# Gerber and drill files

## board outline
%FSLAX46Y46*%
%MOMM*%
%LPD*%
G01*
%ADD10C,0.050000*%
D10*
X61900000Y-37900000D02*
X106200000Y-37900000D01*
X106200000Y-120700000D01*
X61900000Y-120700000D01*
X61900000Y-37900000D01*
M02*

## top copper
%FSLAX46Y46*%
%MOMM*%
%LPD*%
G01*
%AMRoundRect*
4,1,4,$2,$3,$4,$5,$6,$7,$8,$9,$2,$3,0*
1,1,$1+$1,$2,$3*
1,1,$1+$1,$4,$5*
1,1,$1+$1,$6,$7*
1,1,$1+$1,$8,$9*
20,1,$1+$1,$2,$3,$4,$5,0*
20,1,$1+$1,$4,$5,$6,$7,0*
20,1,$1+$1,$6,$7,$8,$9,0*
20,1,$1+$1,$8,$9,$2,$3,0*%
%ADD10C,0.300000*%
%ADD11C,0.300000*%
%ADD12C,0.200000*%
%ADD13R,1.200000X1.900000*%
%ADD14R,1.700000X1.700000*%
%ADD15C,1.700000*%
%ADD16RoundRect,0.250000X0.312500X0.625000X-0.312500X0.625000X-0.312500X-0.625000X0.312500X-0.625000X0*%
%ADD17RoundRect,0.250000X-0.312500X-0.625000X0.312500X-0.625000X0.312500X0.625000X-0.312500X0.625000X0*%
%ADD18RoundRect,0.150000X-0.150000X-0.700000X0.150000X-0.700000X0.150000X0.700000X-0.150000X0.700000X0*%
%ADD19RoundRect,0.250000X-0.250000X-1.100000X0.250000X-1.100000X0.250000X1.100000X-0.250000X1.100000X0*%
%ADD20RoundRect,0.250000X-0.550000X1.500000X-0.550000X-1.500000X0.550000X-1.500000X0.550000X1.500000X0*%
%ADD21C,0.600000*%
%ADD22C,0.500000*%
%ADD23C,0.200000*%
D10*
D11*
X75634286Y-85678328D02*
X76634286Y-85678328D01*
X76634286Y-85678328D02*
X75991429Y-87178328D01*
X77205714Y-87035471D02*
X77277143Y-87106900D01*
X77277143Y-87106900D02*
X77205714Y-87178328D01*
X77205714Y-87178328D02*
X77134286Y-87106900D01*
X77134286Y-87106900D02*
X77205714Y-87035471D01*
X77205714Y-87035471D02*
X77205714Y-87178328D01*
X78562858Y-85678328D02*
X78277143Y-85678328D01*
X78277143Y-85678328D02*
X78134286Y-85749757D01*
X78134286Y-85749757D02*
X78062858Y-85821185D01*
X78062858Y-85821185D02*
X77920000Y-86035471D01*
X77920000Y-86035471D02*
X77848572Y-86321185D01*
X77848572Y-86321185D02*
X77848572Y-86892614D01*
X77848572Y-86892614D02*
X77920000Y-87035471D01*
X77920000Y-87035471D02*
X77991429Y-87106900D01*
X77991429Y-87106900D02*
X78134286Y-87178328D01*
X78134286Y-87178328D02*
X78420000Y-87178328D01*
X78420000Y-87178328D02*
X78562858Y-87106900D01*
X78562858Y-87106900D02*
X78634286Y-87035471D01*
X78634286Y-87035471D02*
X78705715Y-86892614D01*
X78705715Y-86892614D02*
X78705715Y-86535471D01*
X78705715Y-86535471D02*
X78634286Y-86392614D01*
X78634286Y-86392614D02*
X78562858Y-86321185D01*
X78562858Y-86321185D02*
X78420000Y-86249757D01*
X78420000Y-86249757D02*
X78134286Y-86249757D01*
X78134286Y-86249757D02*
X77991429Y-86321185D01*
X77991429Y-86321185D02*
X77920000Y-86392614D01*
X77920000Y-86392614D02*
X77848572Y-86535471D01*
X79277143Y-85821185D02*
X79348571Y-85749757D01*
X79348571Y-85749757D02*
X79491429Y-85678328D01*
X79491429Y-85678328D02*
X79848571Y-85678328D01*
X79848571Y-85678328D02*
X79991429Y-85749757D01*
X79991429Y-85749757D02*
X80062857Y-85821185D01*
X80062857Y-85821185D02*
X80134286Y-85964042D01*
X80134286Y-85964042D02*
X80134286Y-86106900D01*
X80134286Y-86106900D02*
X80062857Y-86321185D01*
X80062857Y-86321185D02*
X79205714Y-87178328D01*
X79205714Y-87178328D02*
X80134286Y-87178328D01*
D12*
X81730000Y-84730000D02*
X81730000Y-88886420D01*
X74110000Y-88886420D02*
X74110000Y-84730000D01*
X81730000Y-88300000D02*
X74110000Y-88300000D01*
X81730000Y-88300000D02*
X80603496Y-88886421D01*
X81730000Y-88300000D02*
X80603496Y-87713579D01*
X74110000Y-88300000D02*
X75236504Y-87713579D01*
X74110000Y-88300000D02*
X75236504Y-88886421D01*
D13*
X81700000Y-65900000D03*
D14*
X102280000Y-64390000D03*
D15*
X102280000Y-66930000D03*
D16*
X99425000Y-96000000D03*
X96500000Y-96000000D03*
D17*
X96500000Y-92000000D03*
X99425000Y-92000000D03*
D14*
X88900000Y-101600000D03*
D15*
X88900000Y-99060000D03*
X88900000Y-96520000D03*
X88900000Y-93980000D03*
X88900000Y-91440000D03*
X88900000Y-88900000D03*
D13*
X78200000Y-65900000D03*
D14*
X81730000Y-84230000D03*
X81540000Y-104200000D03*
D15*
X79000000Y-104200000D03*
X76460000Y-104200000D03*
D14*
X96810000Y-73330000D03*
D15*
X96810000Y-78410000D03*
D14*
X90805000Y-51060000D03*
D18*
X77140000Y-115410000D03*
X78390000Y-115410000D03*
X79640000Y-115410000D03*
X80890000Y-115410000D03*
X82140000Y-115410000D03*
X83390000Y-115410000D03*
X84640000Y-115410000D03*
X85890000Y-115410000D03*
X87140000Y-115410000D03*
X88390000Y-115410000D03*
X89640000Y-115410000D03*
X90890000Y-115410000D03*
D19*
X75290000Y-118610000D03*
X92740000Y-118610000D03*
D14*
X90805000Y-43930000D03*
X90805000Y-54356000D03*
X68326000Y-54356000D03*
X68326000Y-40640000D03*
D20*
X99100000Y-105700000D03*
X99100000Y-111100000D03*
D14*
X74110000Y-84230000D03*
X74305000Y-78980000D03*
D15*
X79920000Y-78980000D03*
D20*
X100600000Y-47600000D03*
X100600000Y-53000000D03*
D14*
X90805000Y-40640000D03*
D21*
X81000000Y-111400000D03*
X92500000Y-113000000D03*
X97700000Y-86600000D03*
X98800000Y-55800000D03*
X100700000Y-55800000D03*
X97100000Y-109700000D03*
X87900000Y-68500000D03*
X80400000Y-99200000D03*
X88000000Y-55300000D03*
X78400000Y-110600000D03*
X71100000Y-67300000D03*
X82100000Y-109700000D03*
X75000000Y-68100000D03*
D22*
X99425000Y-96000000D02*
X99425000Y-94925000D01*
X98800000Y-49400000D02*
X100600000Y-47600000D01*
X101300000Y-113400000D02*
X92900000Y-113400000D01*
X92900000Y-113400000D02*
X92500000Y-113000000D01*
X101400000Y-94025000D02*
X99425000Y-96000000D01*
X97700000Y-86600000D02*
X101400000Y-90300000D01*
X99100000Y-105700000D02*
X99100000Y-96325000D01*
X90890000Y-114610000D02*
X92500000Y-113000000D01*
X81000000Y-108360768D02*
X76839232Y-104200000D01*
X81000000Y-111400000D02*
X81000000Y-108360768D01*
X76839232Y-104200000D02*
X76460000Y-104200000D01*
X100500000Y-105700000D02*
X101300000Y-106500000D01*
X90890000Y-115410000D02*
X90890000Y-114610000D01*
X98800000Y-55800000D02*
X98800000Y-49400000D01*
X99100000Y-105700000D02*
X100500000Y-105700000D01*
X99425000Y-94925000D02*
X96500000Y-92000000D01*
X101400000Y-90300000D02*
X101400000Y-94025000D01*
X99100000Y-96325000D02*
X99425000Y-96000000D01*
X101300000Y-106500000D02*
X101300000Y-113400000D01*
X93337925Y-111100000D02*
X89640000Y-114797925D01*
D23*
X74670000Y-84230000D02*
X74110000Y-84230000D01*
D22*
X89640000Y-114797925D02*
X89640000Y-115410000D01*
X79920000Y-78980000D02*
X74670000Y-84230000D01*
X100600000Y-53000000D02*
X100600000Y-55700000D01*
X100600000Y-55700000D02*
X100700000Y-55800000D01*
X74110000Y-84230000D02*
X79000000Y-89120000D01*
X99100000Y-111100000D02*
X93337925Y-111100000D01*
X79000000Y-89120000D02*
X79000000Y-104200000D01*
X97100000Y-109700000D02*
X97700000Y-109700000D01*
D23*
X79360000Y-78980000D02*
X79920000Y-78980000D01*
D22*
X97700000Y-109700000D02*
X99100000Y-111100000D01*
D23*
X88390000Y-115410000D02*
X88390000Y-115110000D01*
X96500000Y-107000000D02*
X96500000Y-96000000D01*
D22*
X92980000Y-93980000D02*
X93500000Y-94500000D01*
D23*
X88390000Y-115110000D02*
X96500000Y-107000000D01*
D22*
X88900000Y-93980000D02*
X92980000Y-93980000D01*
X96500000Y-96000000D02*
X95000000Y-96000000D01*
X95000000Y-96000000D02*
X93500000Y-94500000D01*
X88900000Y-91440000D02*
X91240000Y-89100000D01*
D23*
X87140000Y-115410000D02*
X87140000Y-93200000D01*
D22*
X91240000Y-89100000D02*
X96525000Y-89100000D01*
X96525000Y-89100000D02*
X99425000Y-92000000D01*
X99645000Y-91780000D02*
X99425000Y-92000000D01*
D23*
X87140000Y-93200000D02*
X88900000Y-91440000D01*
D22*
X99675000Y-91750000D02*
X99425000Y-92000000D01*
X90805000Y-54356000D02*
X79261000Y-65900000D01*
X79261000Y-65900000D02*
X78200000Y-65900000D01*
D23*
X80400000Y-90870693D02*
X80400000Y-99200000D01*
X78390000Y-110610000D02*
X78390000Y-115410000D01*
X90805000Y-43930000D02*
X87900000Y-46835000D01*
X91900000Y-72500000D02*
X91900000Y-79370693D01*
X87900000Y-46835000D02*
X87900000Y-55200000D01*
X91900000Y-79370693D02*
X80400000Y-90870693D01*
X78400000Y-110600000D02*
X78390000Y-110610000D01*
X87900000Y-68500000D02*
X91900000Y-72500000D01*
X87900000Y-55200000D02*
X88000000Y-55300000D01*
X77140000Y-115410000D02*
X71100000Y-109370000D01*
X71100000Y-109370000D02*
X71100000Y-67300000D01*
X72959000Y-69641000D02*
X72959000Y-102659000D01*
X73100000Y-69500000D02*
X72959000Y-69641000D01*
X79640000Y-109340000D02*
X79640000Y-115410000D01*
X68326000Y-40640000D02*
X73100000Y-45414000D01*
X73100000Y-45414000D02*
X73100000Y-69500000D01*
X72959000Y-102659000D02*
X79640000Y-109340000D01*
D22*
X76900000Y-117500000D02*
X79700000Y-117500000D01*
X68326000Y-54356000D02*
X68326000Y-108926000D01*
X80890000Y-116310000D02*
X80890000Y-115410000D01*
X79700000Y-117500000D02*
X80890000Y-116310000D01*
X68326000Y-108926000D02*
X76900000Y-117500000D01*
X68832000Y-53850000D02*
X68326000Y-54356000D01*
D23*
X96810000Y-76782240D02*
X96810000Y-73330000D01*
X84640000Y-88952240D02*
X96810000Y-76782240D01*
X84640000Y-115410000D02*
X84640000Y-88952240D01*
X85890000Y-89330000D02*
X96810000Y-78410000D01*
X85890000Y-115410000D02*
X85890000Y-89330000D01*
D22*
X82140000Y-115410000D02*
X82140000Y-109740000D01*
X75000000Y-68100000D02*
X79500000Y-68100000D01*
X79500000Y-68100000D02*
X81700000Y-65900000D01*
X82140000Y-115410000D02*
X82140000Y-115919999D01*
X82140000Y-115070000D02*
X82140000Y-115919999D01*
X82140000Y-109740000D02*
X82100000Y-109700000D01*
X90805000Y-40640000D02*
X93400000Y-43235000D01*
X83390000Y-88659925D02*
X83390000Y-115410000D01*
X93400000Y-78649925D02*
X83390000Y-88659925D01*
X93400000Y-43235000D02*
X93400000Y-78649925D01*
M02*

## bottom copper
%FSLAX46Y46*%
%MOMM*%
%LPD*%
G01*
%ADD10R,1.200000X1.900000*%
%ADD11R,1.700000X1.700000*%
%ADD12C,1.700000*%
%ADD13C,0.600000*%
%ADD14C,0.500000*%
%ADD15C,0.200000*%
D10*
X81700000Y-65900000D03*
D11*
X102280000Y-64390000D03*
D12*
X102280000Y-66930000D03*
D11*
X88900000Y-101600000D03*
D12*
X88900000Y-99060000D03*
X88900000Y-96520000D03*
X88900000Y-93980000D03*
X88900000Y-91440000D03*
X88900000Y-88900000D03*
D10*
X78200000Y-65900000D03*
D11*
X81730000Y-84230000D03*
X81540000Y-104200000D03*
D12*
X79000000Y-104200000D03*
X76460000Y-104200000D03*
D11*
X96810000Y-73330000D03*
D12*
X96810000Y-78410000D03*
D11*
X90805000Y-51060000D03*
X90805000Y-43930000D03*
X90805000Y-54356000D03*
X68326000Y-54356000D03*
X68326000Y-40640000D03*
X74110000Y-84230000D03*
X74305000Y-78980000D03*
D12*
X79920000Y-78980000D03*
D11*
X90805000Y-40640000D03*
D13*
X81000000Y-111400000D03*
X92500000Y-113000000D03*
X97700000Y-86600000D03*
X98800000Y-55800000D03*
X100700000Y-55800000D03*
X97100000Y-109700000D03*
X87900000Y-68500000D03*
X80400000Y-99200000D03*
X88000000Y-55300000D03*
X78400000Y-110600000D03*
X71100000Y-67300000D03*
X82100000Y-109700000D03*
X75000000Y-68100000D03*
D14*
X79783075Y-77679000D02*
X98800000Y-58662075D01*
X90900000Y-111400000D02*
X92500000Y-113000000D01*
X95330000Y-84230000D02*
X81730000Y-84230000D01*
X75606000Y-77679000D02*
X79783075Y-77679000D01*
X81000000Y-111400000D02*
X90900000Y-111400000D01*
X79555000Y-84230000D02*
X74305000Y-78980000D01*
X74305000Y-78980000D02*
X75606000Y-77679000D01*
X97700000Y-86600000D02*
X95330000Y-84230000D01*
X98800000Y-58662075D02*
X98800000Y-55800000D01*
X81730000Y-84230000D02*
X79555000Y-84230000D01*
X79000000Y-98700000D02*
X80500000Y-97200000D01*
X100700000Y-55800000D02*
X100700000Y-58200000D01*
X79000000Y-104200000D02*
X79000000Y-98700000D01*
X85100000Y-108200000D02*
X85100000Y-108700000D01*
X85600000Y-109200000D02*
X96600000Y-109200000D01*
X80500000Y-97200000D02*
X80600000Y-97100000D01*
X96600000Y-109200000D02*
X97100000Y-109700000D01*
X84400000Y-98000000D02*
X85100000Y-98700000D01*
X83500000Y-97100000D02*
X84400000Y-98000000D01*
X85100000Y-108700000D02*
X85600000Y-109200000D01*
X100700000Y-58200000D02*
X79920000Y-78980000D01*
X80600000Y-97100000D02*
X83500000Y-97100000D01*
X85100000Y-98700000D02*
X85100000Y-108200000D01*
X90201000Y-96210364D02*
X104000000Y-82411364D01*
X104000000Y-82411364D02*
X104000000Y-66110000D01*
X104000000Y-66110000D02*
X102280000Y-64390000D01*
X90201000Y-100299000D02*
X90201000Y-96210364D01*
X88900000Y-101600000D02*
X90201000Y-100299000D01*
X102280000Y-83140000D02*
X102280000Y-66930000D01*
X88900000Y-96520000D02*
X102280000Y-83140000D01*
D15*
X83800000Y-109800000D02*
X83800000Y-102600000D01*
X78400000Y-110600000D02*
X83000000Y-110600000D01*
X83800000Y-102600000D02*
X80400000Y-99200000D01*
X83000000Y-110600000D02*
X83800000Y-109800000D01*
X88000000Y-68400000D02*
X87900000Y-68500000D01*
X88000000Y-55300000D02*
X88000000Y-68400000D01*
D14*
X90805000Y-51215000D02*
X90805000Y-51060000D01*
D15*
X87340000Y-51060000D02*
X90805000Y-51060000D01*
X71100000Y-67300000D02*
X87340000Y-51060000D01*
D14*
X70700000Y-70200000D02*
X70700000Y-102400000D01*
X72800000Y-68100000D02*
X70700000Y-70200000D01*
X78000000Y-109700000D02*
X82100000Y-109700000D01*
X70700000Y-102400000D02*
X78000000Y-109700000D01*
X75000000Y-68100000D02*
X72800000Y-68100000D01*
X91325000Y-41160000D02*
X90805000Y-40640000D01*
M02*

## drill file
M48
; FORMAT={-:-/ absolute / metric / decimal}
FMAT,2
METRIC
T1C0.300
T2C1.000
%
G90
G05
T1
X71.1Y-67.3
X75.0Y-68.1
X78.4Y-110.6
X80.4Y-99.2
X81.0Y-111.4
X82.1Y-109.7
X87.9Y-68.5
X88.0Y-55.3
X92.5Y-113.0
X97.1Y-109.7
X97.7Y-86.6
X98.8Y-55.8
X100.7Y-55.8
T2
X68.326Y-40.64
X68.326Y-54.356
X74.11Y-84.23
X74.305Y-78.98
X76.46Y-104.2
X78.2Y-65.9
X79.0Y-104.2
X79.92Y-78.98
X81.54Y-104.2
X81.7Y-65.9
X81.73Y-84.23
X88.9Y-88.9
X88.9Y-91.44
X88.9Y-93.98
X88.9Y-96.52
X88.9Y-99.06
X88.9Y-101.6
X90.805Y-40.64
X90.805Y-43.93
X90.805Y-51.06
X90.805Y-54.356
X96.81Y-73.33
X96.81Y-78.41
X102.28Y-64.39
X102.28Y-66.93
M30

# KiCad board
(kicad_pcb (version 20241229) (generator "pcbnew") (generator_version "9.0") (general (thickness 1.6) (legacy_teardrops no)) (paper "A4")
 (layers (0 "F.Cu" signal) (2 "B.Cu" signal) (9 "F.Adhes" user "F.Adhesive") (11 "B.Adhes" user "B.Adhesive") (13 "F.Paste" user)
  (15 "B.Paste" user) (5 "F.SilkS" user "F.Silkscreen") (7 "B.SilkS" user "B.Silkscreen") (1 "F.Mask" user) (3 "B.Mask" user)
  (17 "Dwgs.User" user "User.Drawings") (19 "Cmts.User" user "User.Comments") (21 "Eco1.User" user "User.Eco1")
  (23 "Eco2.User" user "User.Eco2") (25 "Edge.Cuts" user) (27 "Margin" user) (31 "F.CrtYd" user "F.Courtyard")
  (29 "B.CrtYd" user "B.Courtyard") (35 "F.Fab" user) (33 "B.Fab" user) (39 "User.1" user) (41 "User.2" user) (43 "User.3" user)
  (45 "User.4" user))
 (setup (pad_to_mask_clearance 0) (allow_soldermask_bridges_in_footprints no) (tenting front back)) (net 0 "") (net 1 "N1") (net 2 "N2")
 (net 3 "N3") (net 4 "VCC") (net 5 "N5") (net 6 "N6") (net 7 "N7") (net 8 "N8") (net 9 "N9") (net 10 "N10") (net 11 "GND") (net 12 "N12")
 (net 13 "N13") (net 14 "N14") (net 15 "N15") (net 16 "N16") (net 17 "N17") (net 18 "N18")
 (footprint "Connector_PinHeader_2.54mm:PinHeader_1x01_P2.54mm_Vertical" (layer "F.Cu") (at 81.7 65.9 90)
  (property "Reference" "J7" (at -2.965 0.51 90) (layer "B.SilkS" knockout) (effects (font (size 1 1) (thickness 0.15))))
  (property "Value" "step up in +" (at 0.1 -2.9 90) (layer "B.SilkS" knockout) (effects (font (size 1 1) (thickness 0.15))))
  (pad "1" thru_hole rect (at 0 0 90) (size 1.9 1.2) (drill 1) (layers "*.Cu" "*.Mask") (remove_unused_layers no) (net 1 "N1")))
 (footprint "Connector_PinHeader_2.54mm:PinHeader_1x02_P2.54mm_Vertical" (layer "F.Cu") (at 102.28 64.39)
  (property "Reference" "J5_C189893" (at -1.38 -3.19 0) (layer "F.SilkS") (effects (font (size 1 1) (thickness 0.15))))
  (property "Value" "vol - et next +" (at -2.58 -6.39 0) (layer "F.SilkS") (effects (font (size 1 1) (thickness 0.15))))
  (pad "1" thru_hole rect (at 0 0) (size 1.7 1.7) (drill 1) (layers "*.Cu" "*.Mask") (remove_unused_layers no) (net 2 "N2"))
  (pad "2" thru_hole circle (at 0 2.54) (size 1.7 1.7) (drill 1) (layers "*.Cu" "*.Mask") (remove_unused_layers no) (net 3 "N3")))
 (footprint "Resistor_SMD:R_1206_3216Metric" (layer "F.Cu") (at 97.9625 96 180)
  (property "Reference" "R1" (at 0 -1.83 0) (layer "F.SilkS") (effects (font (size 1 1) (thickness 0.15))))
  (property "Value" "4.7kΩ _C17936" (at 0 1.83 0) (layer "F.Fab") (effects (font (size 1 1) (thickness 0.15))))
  (pad "1" smd roundrect (at -1.4625 0 180) (size 1.125 1.75) (layers "F.Cu" "F.Mask" "F.Paste") (roundrect_rratio 0.222222) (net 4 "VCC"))
  (pad "2" smd roundrect (at 1.4625 0 180) (size 1.125 1.75) (layers "F.Cu" "F.Mask" "F.Paste") (roundrect_rratio 0.222222) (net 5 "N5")))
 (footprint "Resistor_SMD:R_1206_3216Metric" (layer "F.Cu") (at 97.9625 92)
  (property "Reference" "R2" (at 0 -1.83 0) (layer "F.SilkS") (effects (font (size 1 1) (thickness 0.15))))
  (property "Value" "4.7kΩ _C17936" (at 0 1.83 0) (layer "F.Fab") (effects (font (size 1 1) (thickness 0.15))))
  (pad "1" smd roundrect (at -1.4625 0) (size 1.125 1.75) (layers "F.Cu" "F.Mask" "F.Paste") (roundrect_rratio 0.222222) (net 4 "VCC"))
  (pad "2" smd roundrect (at 1.4625 0) (size 1.125 1.75) (layers "F.Cu" "F.Mask" "F.Paste") (roundrect_rratio 0.222222) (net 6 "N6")))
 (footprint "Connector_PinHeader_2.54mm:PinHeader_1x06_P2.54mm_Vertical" (layer "F.Cu") (at 88.9 101.6 180)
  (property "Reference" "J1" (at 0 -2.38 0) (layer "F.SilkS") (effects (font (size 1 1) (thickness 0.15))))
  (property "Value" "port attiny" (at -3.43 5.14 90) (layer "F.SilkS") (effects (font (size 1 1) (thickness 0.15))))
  (pad "1" thru_hole rect (at 0 0 180) (size 1.7 1.7) (drill 1) (layers "*.Cu" "*.Mask") (remove_unused_layers no) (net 2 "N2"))
  (pad "2" thru_hole circle (at 0 2.54 180) (size 1.7 1.7) (drill 1) (layers "*.Cu" "*.Mask") (remove_unused_layers no) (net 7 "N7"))
  (pad "3" thru_hole circle (at 0 5.08 180) (size 1.7 1.7) (drill 1) (layers "*.Cu" "*.Mask") (remove_unused_layers no) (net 3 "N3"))
  (pad "4" thru_hole circle (at 0 7.62 180) (size 1.7 1.7) (drill 1) (layers "*.Cu" "*.Mask") (remove_unused_layers no) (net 5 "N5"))
  (pad "5" thru_hole circle (at 0 10.16 180) (size 1.7 1.7) (drill 1) (layers "*.Cu" "*.Mask") (remove_unused_layers no) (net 6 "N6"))
  (pad "6" thru_hole circle (at 0 12.7 180) (size 1.7 1.7) (drill 1) (layers "*.Cu" "*.Mask") (remove_unused_layers no) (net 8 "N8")))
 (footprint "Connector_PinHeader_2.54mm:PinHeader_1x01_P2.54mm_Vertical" (layer "F.Cu") (at 78.1 65.9 90)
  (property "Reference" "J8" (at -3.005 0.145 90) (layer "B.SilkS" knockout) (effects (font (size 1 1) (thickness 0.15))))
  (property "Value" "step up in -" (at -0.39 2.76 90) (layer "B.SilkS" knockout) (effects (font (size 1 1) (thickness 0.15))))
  (pad "1" thru_hole rect (at 0 0.1 90) (size 1.9 1.2) (drill 1) (layers "*.Cu" "*.Mask") (remove_unused_layers no) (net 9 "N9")))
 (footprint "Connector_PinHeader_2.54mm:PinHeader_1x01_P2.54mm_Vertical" (layer "F.Cu") (at 81.73 84.23)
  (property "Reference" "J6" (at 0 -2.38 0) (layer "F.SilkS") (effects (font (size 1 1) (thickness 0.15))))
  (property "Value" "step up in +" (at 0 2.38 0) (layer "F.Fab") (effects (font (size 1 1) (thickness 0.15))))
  (pad "1" thru_hole rect (at 0 0) (size 1.7 1.7) (drill 1) (layers "*.Cu" "*.Mask") (remove_unused_layers no) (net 4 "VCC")
   (padstack (mode custom) (layer "B.Cu" (shape rect) (size 1.7 1.7) (zone_connect -1)))))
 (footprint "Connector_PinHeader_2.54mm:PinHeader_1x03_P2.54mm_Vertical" (layer "F.Cu") (at 81.54 104.2 -90)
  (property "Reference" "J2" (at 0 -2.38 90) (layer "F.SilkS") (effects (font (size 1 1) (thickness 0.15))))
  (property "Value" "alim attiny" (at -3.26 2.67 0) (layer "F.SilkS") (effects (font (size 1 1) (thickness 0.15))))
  (pad "1" thru_hole rect (at 0 0 270) (size 1.7 1.7) (drill 1) (layers "*.Cu" "*.Mask") (remove_unused_layers no) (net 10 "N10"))
  (pad "2" thru_hole circle (at 0 2.54 270) (size 1.7 1.7) (drill 1) (layers "*.Cu" "*.Mask") (remove_unused_layers no) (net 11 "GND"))
  (pad "3" thru_hole circle (at 0 5.08 270) (size 1.7 1.7) (drill 1) (layers "*.Cu" "*.Mask") (remove_unused_layers no) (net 4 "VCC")))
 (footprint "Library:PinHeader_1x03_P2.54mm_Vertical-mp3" (layer "F.Cu") (at 96.81 73.33)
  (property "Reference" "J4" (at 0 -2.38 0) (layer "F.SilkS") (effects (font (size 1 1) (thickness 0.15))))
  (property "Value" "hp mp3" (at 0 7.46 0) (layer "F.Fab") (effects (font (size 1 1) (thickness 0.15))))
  (pad "1" thru_hole rect (at 0 0) (size 1.7 1.7) (drill 1) (layers "*.Cu" "*.Mask") (remove_unused_layers no) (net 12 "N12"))
  (pad "2" thru_hole circle (at 0 5.08) (size 1.7 1.7) (drill 1) (layers "*.Cu" "*.Mask") (remove_unused_layers no) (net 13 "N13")))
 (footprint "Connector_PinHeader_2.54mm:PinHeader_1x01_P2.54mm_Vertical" (layer "F.Cu") (at 90.805 51.06)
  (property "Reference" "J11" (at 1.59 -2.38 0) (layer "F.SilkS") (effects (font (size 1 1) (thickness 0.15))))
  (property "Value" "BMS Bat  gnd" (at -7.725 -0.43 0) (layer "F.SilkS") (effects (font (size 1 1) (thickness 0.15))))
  (pad "1" thru_hole rect (at 0 0) (size 1.7 1.7) (drill 1) (layers "*.Cu" "*.Mask") (remove_unused_layers no) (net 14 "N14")))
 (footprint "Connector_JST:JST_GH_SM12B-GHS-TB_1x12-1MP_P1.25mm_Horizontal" (layer "F.Cu") (at 84.015 117.26)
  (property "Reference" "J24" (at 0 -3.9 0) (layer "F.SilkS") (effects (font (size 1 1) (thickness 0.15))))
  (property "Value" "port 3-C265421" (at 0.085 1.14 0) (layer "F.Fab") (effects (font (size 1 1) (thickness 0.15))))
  (pad "1" smd roundrect (at -6.875 -1.85) (size 0.6 1.7) (layers "F.Cu" "F.Mask" "F.Paste") (roundrect_rratio 0.25) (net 14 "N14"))
  (pad "2" smd roundrect (at -5.625 -1.85) (size 0.6 1.7) (layers "F.Cu" "F.Mask" "F.Paste") (roundrect_rratio 0.25) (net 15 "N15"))
  (pad "3" smd roundrect (at -4.375 -1.85) (size 0.6 1.7) (layers "F.Cu" "F.Mask" "F.Paste") (roundrect_rratio 0.25) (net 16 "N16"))
  (pad "4" smd roundrect (at -3.125 -1.85) (size 0.6 1.7) (layers "F.Cu" "F.Mask" "F.Paste") (roundrect_rratio 0.25) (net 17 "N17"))
  (pad "5" smd roundrect (at -1.875 -1.85) (size 0.6 1.7) (layers "F.Cu" "F.Mask" "F.Paste") (roundrect_rratio 0.25) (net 1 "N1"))
  (pad "6" smd roundrect (at -0.625 -1.85) (size 0.6 1.7) (layers "F.Cu" "F.Mask" "F.Paste") (roundrect_rratio 0.25) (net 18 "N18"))
  (pad "7" smd roundrect (at 0.625 -1.85) (size 0.6 1.7) (layers "F.Cu" "F.Mask" "F.Paste") (roundrect_rratio 0.25) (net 12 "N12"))
  (pad "8" smd roundrect (at 1.875 -1.85) (size 0.6 1.7) (layers "F.Cu" "F.Mask" "F.Paste") (roundrect_rratio 0.25) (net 13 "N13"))
  (pad "9" smd roundrect (at 3.125 -1.85) (size 0.6 1.7) (layers "F.Cu" "F.Mask" "F.Paste") (roundrect_rratio 0.25) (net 6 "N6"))
  (pad "10" smd roundrect (at 4.375 -1.85) (size 0.6 1.7) (layers "F.Cu" "F.Mask" "F.Paste") (roundrect_rratio 0.25) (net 5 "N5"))
  (pad "11" smd roundrect (at 5.625 -1.85) (size 0.6 1.7) (layers "F.Cu" "F.Mask" "F.Paste") (roundrect_rratio 0.25) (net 11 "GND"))
  (pad "12" smd roundrect (at 6.875 -1.85) (size 0.6 1.7) (layers "F.Cu" "F.Mask" "F.Paste") (roundrect_rratio 0.25) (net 4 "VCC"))
  (pad "MP" smd roundrect (at -8.725 1.35) (size 1 2.7) (layers "F.Cu" "F.Mask" "F.Paste") (roundrect_rratio 0.25))
  (pad "MP" smd roundrect (at 8.725 1.35) (size 1 2.7) (layers "F.Cu" "F.Mask" "F.Paste") (roundrect_rratio 0.25)))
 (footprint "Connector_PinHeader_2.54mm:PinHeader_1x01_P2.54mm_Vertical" (layer "F.Cu") (at 90.805 43.93)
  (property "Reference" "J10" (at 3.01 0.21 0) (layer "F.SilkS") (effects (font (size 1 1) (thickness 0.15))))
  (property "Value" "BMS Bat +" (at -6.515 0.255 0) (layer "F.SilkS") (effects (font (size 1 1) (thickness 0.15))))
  (pad "1" thru_hole rect (at 0 0) (size 1.7 1.7) (drill 1) (layers "*.Cu" "*.Mask") (remove_unused_layers no) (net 15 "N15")))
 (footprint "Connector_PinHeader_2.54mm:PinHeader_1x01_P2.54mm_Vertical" (layer "F.Cu") (at 90.805 54.356)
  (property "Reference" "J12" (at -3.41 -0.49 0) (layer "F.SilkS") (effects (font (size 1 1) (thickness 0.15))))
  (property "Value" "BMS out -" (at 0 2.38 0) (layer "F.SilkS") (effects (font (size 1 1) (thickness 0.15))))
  (pad "1" thru_hole rect (at 0 0) (size 1.7 1.7) (drill 1) (layers "*.Cu" "*.Mask") (remove_unused_layers no) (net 9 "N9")))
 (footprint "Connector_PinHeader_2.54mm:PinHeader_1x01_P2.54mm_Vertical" (layer "F.Cu") (at 68.326 54.356)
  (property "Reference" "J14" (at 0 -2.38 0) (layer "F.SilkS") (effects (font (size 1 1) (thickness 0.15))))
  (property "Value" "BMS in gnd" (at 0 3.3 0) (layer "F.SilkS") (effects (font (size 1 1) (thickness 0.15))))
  (pad "1" thru_hole rect (at 0 0) (size 1.7 1.7) (drill 1) (layers "*.Cu" "*.Mask") (remove_unused_layers no) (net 17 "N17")))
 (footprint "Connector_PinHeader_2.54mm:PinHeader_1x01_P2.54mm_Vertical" (layer "F.Cu") (at 68.326 40.64)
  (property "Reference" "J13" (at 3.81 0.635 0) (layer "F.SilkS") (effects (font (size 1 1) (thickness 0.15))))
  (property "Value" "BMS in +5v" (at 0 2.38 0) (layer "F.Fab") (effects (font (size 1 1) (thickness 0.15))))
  (pad "1" thru_hole rect (at 0 0) (size 1.7 1.7) (drill 1) (layers "*.Cu" "*.Mask") (remove_unused_layers no) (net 16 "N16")))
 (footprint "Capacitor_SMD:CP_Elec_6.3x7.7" (layer "F.Cu") (at 99.1 108.4 -90)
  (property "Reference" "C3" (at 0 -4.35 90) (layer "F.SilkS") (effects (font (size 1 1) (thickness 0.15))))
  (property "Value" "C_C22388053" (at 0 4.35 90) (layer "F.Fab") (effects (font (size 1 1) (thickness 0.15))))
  (pad "1" smd roundrect (at -2.7 0 270) (size 3.5 1.6) (layers "F.Cu" "F.Mask" "F.Paste") (roundrect_rratio 0.15625) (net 4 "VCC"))
  (pad "2" smd roundrect (at 2.7 0 270) (size 3.5 1.6) (layers "F.Cu" "F.Mask" "F.Paste") (roundrect_rratio 0.15625) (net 11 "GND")))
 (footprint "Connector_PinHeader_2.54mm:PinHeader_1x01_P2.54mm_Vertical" (layer "F.Cu") (at 74.11 84.23)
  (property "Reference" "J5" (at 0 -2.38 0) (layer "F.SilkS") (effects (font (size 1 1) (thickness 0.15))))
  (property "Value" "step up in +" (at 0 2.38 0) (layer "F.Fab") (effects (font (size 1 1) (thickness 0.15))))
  (pad "1" thru_hole rect (at 0 0) (size 1.7 1.7) (drill 1) (layers "*.Cu" "*.Mask") (remove_unused_layers no) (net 11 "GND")))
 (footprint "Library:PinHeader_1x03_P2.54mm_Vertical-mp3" (layer "F.Cu") (at 74.84 78.98 90)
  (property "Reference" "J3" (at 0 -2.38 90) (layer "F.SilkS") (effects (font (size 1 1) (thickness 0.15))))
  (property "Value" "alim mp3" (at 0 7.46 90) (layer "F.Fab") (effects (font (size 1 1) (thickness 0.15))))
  (pad "1" thru_hole rect (at 0 -0.535 90) (size 1.7 1.7) (drill 1) (layers "*.Cu" "*.Mask") (remove_unused_layers no) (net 4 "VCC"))
  (pad "2" thru_hole circle (at 0 5.08 90) (size 1.7 1.7) (drill 1) (layers "*.Cu" "*.Mask") (remove_unused_layers no) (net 11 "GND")))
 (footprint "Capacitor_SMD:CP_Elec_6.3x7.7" (layer "F.Cu") (at 100.6 50.3 -90)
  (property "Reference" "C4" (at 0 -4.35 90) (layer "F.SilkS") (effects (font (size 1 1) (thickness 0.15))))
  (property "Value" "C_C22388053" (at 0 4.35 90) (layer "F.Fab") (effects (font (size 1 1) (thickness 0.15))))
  (pad "1" smd roundrect (at -2.7 0 270) (size 3.5 1.6) (layers "F.Cu" "F.Mask" "F.Paste") (roundrect_rratio 0.15625) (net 4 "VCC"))
  (pad "2" smd roundrect (at 2.7 0 270) (size 3.5 1.6) (layers "F.Cu" "F.Mask" "F.Paste") (roundrect_rratio 0.15625) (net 11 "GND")))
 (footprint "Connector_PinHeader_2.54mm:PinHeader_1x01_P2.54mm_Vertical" (layer "F.Cu") (at 90.805 40.64)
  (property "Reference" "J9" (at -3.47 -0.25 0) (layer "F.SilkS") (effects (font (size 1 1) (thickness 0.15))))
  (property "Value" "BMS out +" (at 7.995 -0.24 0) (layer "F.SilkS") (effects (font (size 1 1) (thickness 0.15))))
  (pad "1" thru_hole rect (at 0 0) (size 1.7 1.7) (drill 1) (layers "*.Cu" "*.Mask") (remove_unused_layers no) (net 18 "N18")))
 (gr_rect (start 61.9 37.9) (end 106.2 120.7) (stroke (width 0.05) (type solid)) (fill no) (layer "Edge.Cuts"))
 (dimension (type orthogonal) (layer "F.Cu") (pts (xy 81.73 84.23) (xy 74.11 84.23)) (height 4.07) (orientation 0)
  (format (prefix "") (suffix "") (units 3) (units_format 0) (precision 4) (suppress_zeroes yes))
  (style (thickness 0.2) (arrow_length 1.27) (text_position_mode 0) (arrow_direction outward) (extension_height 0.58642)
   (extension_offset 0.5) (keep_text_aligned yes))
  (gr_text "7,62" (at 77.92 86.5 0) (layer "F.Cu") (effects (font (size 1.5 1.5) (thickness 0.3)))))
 (segment (start 99.425 96) (end 99.425 94.925) (width 0.5) (layer "F.Cu") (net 4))
 (segment (start 98.8 49.4) (end 100.6 47.6) (width 0.5) (layer "F.Cu") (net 4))
 (segment (start 101.3 113.4) (end 92.9 113.4) (width 0.5) (layer "F.Cu") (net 4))
 (segment (start 92.9 113.4) (end 92.5 113) (width 0.5) (layer "F.Cu") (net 4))
 (segment (start 101.4 94.025) (end 99.425 96) (width 0.5) (layer "F.Cu") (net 4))
 (segment (start 97.7 86.6) (end 101.4 90.3) (width 0.5) (layer "F.Cu") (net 4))
 (segment (start 99.1 105.7) (end 99.1 96.325) (width 0.5) (layer "F.Cu") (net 4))
 (segment (start 90.89 114.61) (end 92.5 113) (width 0.5) (layer "F.Cu") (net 4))
 (segment (start 81 108.360768) (end 76.839232 104.2) (width 0.5) (layer "F.Cu") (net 4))
 (segment (start 81 111.4) (end 81 108.360768) (width 0.5) (layer "F.Cu") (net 4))
 (segment (start 76.839232 104.2) (end 76.46 104.2) (width 0.5) (layer "F.Cu") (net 4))
 (segment (start 100.5 105.7) (end 101.3 106.5) (width 0.5) (layer "F.Cu") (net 4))
 (segment (start 90.89 115.41) (end 90.89 114.61) (width 0.5) (layer "F.Cu") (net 4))
 (segment (start 98.8 55.8) (end 98.8 49.4) (width 0.5) (layer "F.Cu") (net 4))
 (segment (start 99.1 105.7) (end 100.5 105.7) (width 0.5) (layer "F.Cu") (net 4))
 (segment (start 99.425 94.925) (end 96.5 92) (width 0.5) (layer "F.Cu") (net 4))
 (segment (start 101.4 90.3) (end 101.4 94.025) (width 0.5) (layer "F.Cu") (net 4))
 (segment (start 99.1 96.325) (end 99.425 96) (width 0.5) (layer "F.Cu") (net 4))
 (segment (start 101.3 106.5) (end 101.3 113.4) (width 0.5) (layer "F.Cu") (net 4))
 (via (at 81 111.4) (size 0.6) (drill 0.3) (layers "F.Cu" "B.Cu") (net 4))
 (via (at 92.5 113) (size 0.6) (drill 0.3) (layers "F.Cu" "B.Cu") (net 4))
 (via (at 97.7 86.6) (size 0.6) (drill 0.3) (layers "F.Cu" "B.Cu") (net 4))
 (via (at 98.8 55.8) (size 0.6) (drill 0.3) (layers "F.Cu" "B.Cu") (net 4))
 (segment (start 79.783075 77.679) (end 98.8 58.662075) (width 0.5) (layer "B.Cu") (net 4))
 (segment (start 90.9 111.4) (end 92.5 113) (width 0.5) (layer "B.Cu") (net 4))
 (segment (start 95.33 84.23) (end 81.73 84.23) (width 0.5) (layer "B.Cu") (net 4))
 (segment (start 75.606 77.679) (end 79.783075 77.679) (width 0.5) (layer "B.Cu") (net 4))
 (segment (start 81 111.4) (end 90.9 111.4) (width 0.5) (layer "B.Cu") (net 4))
 (segment (start 79.555 84.23) (end 74.305 78.98) (width 0.5) (layer "B.Cu") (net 4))
 (segment (start 74.305 78.98) (end 75.606 77.679) (width 0.5) (layer "B.Cu") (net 4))
 (segment (start 97.7 86.6) (end 95.33 84.23) (width 0.5) (layer "B.Cu") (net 4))
 (segment (start 98.8 58.662075) (end 98.8 55.8) (width 0.5) (layer "B.Cu") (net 4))
 (segment (start 81.73 84.23) (end 79.555 84.23) (width 0.5) (layer "B.Cu") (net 4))
 (segment (start 93.337925 111.1) (end 89.64 114.797925) (width 0.5) (layer "F.Cu") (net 11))
 (segment (start 74.67 84.23) (end 74.11 84.23) (width 0.2) (layer "F.Cu") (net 11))
 (segment (start 89.64 114.797925) (end 89.64 115.41) (width 0.5) (layer "F.Cu") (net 11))
 (segment (start 79.92 78.98) (end 74.67 84.23) (width 0.5) (layer "F.Cu") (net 11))
 (segment (start 100.6 53) (end 100.6 55.7) (width 0.5) (layer "F.Cu") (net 11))
 (segment (start 100.6 55.7) (end 100.7 55.8) (width 0.5) (layer "F.Cu") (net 11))
 (segment (start 74.11 84.23) (end 79 89.12) (width 0.5) (layer "F.Cu") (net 11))
 (segment (start 99.1 111.1) (end 93.337925 111.1) (width 0.5) (layer "F.Cu") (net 11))
 (segment (start 79 89.12) (end 79 104.2) (width 0.5) (layer "F.Cu") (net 11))
 (segment (start 97.1 109.7) (end 97.7 109.7) (width 0.5) (layer "F.Cu") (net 11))
 (segment (start 79.36 78.98) (end 79.92 78.98) (width 0.2) (layer "F.Cu") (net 11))
 (segment (start 97.7 109.7) (end 99.1 111.1) (width 0.5) (layer "F.Cu") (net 11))
 (via (at 100.7 55.8) (size 0.6) (drill 0.3) (layers "F.Cu" "B.Cu") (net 11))
 (via (at 97.1 109.7) (size 0.6) (drill 0.3) (layers "F.Cu" "B.Cu") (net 11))
 (segment (start 79 98.7) (end 80.5 97.2) (width 0.5) (layer "B.Cu") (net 11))
 (segment (start 100.7 55.8) (end 100.7 58.2) (width 0.5) (layer "B.Cu") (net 11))
 (segment (start 79 104.2) (end 79 98.7) (width 0.5) (layer "B.Cu") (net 11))
 (segment (start 85.1 108.2) (end 85.1 108.7) (width 0.5) (layer "B.Cu") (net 11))
 (segment (start 85.6 109.2) (end 96.6 109.2) (width 0.5) (layer "B.Cu") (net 11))
 (segment (start 80.5 97.2) (end 80.6 97.1) (width 0.5) (layer "B.Cu") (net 11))
 (segment (start 96.6 109.2) (end 97.1 109.7) (width 0.5) (layer "B.Cu") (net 11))
 (segment (start 84.4 98) (end 85.1 98.7) (width 0.5) (layer "B.Cu") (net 11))
 (segment (start 83.5 97.1) (end 84.4 98) (width 0.5) (layer "B.Cu") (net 11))
 (segment (start 85.1 108.7) (end 85.6 109.2) (width 0.5) (layer "B.Cu") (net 11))
 (segment (start 100.7 58.2) (end 79.92 78.98) (width 0.5) (layer "B.Cu") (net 11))
 (segment (start 80.6 97.1) (end 83.5 97.1) (width 0.5) (layer "B.Cu") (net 11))
 (segment (start 85.1 98.7) (end 85.1 108.2) (width 0.5) (layer "B.Cu") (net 11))
 (segment (start 88.39 115.41) (end 88.39 115.11) (width 0.2) (layer "F.Cu") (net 5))
 (segment (start 96.5 107) (end 96.5 96) (width 0.2) (layer "F.Cu") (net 5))
 (segment (start 92.98 93.98) (end 93.5 94.5) (width 0.5) (layer "F.Cu") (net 5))
 (segment (start 88.39 115.11) (end 96.5 107) (width 0.2) (layer "F.Cu") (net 5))
 (segment (start 88.9 93.98) (end 92.98 93.98) (width 0.5) (layer "F.Cu") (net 5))
 (segment (start 96.5 96) (end 95 96) (width 0.5) (layer "F.Cu") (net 5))
 (segment (start 95 96) (end 93.5 94.5) (width 0.5) (layer "F.Cu") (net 5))
 (segment (start 88.9 91.44) (end 91.24 89.1) (width 0.5) (layer "F.Cu") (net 6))
 (segment (start 87.14 115.41) (end 87.14 93.2) (width 0.2) (layer "F.Cu") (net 6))
 (segment (start 91.24 89.1) (end 96.525 89.1) (width 0.5) (layer "F.Cu") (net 6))
 (segment (start 96.525 89.1) (end 99.425 92) (width 0.5) (layer "F.Cu") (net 6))
 (segment (start 99.645 91.78) (end 99.425 92) (width 0.5) (layer "F.Cu") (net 6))
 (segment (start 87.14 93.2) (end 88.9 91.44) (width 0.2) (layer "F.Cu") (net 6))
 (segment (start 99.675 91.75) (end 99.425 92) (width 0.5) (layer "F.Cu") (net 6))
 (segment (start 90.201 96.210364) (end 104 82.411364) (width 0.5) (layer "B.Cu") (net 2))
 (segment (start 104 82.411364) (end 104 66.11) (width 0.5) (layer "B.Cu") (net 2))
 (segment (start 104 66.11) (end 102.28 64.39) (width 0.5) (layer "B.Cu") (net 2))
 (segment (start 90.201 100.299) (end 90.201 96.210364) (width 0.5) (layer "B.Cu") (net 2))
 (segment (start 88.9 101.6) (end 90.201 100.299) (width 0.5) (layer "B.Cu") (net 2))
 (segment (start 102.28 83.14) (end 102.28 66.93) (width 0.5) (layer "B.Cu") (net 3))
 (segment (start 88.9 96.52) (end 102.28 83.14) (width 0.5) (layer "B.Cu") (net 3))
 (segment (start 90.805 54.356) (end 79.261 65.9) (width 0.5) (layer "F.Cu") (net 9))
 (segment (start 79.261 65.9) (end 78.2 65.9) (width 0.5) (layer "F.Cu") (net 9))
 (segment (start 80.4 90.870693) (end 80.4 99.2) (width 0.2) (layer "F.Cu") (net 15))
 (segment (start 78.39 110.61) (end 78.39 115.41) (width 0.2) (layer "F.Cu") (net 15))
 (segment (start 90.805 43.93) (end 87.9 46.835) (width 0.2) (layer "F.Cu") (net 15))
 (segment (start 91.9 72.5) (end 91.9 79.370693) (width 0.2) (layer "F.Cu") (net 15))
 (segment (start 87.9 46.835) (end 87.9 55.2) (width 0.2) (layer "F.Cu") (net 15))
 (segment (start 91.9 79.370693) (end 80.4 90.870693) (width 0.2) (layer "F.Cu") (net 15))
 (segment (start 78.4 110.6) (end 78.39 110.61) (width 0.2) (layer "F.Cu") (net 15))
 (segment (start 87.9 68.5) (end 91.9 72.5) (width 0.2) (layer "F.Cu") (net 15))
 (segment (start 87.9 55.2) (end 88 55.3) (width 0.2) (layer "F.Cu") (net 15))
 (via (at 87.9 68.5) (size 0.6) (drill 0.3) (layers "F.Cu" "B.Cu") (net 15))
 (via (at 80.4 99.2) (size 0.6) (drill 0.3) (layers "F.Cu" "B.Cu") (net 15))
 (via (at 88 55.3) (size 0.6) (drill 0.3) (layers "F.Cu" "B.Cu") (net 15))
 (via (at 78.4 110.6) (size 0.6) (drill 0.3) (layers "F.Cu" "B.Cu") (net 15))
 (segment (start 83.8 109.8) (end 83.8 102.6) (width 0.2) (layer "B.Cu") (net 15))
 (segment (start 78.4 110.6) (end 83 110.6) (width 0.2) (layer "B.Cu") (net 15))
 (segment (start 83.8 102.6) (end 80.4 99.2) (width 0.2) (layer "B.Cu") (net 15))
 (segment (start 83 110.6) (end 83.8 109.8) (width 0.2) (layer "B.Cu") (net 15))
 (segment (start 88 68.4) (end 87.9 68.5) (width 0.2) (layer "B.Cu") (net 15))
 (segment (start 88 55.3) (end 88 68.4) (width 0.2) (layer "B.Cu") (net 15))
 (segment (start 77.14 115.41) (end 71.1 109.37) (width 0.2) (layer "F.Cu") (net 14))
 (segment (start 71.1 109.37) (end 71.1 67.3) (width 0.2) (layer "F.Cu") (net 14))
 (via (at 71.1 67.3) (size 0.6) (drill 0.3) (layers "F.Cu" "B.Cu") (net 14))
 (segment (start 90.805 51.215) (end 90.805 51.06) (width 0.5) (layer "B.Cu") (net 14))
 (segment (start 87.34 51.06) (end 90.805 51.06) (width 0.2) (layer "B.Cu") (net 14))
 (segment (start 71.1 67.3) (end 87.34 51.06) (width 0.2) (layer "B.Cu") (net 14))
 (segment (start 72.959 69.641) (end 72.959 102.659) (width 0.2) (layer "F.Cu") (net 16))
 (segment (start 73.1 69.5) (end 72.959 69.641) (width 0.2) (layer "F.Cu") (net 16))
 (segment (start 79.64 109.34) (end 79.64 115.41) (width 0.2) (layer "F.Cu") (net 16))
 (segment (start 68.326 40.64) (end 73.1 45.414) (width 0.2) (layer "F.Cu") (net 16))
 (segment (start 73.1 45.414) (end 73.1 69.5) (width 0.2) (layer "F.Cu") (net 16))
 (segment (start 72.959 102.659) (end 79.64 109.34) (width 0.2) (layer "F.Cu") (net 16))
 (segment (start 76.9 117.5) (end 79.7 117.5) (width 0.5) (layer "F.Cu") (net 17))
 (segment (start 68.326 54.356) (end 68.326 108.926) (width 0.5) (layer "F.Cu") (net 17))
 (segment (start 80.89 116.31) (end 80.89 115.41) (width 0.5) (layer "F.Cu") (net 17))
 (segment (start 79.7 117.5) (end 80.89 116.31) (width 0.5) (layer "F.Cu") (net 17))
 (segment (start 68.326 108.926) (end 76.9 117.5) (width 0.5) (layer "F.Cu") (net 17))
 (segment (start 68.832 53.85) (end 68.326 54.356) (width 0.5) (layer "F.Cu") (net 17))
 (segment (start 96.81 76.78224) (end 96.81 73.33) (width 0.2) (layer "F.Cu") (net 12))
 (segment (start 84.64 88.95224) (end 96.81 76.78224) (width 0.2) (layer "F.Cu") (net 12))
 (segment (start 84.64 115.41) (end 84.64 88.95224) (width 0.2) (layer "F.Cu") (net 12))
 (segment (start 85.89 89.33) (end 96.81 78.41) (width 0.2) (layer "F.Cu") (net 13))
 (segment (start 85.89 115.41) (end 85.89 89.33) (width 0.2) (layer "F.Cu") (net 13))
 (segment (start 82.14 115.41) (end 82.14 109.74) (width 0.5) (layer "F.Cu") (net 1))
 (segment (start 75 68.1) (end 79.5 68.1) (width 0.5) (layer "F.Cu") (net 1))
 (segment (start 79.5 68.1) (end 81.7 65.9) (width 0.5) (layer "F.Cu") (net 1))
 (segment (start 82.14 115.41) (end 82.14 115.919999) (width 0.5) (layer "F.Cu") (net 1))
 (segment (start 82.14 115.07) (end 82.14 115.919999) (width 0.5) (layer "F.Cu") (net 1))
 (segment (start 82.14 109.74) (end 82.1 109.7) (width 0.5) (layer "F.Cu") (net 1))
 (via (at 82.1 109.7) (size 0.6) (drill 0.3) (layers "F.Cu" "B.Cu") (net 1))
 (via (at 75 68.1) (size 0.6) (drill 0.3) (layers "F.Cu" "B.Cu") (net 1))
 (segment (start 70.7 70.2) (end 70.7 102.4) (width 0.5) (layer "B.Cu") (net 1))
 (segment (start 72.8 68.1) (end 70.7 70.2) (width 0.5) (layer "B.Cu") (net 1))
 (segment (start 78 109.7) (end 82.1 109.7) (width 0.5) (layer "B.Cu") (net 1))
 (segment (start 70.7 102.4) (end 78 109.7) (width 0.5) (layer "B.Cu") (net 1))
 (segment (start 75 68.1) (end 72.8 68.1) (width 0.5) (layer "B.Cu") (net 1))
 (segment (start 90.805 40.64) (end 93.4 43.235) (width 0.5) (layer "F.Cu") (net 18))
 (segment (start 83.39 88.659925) (end 83.39 115.41) (width 0.5) (layer "F.Cu") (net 18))
 (segment (start 93.4 78.649925) (end 83.39 88.659925) (width 0.5) (layer "F.Cu") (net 18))
 (segment (start 93.4 43.235) (end 93.4 78.649925) (width 0.5) (layer "F.Cu") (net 18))
 (segment (start 91.325 41.16) (end 90.805 40.64) (width 0.5) (layer "B.Cu") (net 18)))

